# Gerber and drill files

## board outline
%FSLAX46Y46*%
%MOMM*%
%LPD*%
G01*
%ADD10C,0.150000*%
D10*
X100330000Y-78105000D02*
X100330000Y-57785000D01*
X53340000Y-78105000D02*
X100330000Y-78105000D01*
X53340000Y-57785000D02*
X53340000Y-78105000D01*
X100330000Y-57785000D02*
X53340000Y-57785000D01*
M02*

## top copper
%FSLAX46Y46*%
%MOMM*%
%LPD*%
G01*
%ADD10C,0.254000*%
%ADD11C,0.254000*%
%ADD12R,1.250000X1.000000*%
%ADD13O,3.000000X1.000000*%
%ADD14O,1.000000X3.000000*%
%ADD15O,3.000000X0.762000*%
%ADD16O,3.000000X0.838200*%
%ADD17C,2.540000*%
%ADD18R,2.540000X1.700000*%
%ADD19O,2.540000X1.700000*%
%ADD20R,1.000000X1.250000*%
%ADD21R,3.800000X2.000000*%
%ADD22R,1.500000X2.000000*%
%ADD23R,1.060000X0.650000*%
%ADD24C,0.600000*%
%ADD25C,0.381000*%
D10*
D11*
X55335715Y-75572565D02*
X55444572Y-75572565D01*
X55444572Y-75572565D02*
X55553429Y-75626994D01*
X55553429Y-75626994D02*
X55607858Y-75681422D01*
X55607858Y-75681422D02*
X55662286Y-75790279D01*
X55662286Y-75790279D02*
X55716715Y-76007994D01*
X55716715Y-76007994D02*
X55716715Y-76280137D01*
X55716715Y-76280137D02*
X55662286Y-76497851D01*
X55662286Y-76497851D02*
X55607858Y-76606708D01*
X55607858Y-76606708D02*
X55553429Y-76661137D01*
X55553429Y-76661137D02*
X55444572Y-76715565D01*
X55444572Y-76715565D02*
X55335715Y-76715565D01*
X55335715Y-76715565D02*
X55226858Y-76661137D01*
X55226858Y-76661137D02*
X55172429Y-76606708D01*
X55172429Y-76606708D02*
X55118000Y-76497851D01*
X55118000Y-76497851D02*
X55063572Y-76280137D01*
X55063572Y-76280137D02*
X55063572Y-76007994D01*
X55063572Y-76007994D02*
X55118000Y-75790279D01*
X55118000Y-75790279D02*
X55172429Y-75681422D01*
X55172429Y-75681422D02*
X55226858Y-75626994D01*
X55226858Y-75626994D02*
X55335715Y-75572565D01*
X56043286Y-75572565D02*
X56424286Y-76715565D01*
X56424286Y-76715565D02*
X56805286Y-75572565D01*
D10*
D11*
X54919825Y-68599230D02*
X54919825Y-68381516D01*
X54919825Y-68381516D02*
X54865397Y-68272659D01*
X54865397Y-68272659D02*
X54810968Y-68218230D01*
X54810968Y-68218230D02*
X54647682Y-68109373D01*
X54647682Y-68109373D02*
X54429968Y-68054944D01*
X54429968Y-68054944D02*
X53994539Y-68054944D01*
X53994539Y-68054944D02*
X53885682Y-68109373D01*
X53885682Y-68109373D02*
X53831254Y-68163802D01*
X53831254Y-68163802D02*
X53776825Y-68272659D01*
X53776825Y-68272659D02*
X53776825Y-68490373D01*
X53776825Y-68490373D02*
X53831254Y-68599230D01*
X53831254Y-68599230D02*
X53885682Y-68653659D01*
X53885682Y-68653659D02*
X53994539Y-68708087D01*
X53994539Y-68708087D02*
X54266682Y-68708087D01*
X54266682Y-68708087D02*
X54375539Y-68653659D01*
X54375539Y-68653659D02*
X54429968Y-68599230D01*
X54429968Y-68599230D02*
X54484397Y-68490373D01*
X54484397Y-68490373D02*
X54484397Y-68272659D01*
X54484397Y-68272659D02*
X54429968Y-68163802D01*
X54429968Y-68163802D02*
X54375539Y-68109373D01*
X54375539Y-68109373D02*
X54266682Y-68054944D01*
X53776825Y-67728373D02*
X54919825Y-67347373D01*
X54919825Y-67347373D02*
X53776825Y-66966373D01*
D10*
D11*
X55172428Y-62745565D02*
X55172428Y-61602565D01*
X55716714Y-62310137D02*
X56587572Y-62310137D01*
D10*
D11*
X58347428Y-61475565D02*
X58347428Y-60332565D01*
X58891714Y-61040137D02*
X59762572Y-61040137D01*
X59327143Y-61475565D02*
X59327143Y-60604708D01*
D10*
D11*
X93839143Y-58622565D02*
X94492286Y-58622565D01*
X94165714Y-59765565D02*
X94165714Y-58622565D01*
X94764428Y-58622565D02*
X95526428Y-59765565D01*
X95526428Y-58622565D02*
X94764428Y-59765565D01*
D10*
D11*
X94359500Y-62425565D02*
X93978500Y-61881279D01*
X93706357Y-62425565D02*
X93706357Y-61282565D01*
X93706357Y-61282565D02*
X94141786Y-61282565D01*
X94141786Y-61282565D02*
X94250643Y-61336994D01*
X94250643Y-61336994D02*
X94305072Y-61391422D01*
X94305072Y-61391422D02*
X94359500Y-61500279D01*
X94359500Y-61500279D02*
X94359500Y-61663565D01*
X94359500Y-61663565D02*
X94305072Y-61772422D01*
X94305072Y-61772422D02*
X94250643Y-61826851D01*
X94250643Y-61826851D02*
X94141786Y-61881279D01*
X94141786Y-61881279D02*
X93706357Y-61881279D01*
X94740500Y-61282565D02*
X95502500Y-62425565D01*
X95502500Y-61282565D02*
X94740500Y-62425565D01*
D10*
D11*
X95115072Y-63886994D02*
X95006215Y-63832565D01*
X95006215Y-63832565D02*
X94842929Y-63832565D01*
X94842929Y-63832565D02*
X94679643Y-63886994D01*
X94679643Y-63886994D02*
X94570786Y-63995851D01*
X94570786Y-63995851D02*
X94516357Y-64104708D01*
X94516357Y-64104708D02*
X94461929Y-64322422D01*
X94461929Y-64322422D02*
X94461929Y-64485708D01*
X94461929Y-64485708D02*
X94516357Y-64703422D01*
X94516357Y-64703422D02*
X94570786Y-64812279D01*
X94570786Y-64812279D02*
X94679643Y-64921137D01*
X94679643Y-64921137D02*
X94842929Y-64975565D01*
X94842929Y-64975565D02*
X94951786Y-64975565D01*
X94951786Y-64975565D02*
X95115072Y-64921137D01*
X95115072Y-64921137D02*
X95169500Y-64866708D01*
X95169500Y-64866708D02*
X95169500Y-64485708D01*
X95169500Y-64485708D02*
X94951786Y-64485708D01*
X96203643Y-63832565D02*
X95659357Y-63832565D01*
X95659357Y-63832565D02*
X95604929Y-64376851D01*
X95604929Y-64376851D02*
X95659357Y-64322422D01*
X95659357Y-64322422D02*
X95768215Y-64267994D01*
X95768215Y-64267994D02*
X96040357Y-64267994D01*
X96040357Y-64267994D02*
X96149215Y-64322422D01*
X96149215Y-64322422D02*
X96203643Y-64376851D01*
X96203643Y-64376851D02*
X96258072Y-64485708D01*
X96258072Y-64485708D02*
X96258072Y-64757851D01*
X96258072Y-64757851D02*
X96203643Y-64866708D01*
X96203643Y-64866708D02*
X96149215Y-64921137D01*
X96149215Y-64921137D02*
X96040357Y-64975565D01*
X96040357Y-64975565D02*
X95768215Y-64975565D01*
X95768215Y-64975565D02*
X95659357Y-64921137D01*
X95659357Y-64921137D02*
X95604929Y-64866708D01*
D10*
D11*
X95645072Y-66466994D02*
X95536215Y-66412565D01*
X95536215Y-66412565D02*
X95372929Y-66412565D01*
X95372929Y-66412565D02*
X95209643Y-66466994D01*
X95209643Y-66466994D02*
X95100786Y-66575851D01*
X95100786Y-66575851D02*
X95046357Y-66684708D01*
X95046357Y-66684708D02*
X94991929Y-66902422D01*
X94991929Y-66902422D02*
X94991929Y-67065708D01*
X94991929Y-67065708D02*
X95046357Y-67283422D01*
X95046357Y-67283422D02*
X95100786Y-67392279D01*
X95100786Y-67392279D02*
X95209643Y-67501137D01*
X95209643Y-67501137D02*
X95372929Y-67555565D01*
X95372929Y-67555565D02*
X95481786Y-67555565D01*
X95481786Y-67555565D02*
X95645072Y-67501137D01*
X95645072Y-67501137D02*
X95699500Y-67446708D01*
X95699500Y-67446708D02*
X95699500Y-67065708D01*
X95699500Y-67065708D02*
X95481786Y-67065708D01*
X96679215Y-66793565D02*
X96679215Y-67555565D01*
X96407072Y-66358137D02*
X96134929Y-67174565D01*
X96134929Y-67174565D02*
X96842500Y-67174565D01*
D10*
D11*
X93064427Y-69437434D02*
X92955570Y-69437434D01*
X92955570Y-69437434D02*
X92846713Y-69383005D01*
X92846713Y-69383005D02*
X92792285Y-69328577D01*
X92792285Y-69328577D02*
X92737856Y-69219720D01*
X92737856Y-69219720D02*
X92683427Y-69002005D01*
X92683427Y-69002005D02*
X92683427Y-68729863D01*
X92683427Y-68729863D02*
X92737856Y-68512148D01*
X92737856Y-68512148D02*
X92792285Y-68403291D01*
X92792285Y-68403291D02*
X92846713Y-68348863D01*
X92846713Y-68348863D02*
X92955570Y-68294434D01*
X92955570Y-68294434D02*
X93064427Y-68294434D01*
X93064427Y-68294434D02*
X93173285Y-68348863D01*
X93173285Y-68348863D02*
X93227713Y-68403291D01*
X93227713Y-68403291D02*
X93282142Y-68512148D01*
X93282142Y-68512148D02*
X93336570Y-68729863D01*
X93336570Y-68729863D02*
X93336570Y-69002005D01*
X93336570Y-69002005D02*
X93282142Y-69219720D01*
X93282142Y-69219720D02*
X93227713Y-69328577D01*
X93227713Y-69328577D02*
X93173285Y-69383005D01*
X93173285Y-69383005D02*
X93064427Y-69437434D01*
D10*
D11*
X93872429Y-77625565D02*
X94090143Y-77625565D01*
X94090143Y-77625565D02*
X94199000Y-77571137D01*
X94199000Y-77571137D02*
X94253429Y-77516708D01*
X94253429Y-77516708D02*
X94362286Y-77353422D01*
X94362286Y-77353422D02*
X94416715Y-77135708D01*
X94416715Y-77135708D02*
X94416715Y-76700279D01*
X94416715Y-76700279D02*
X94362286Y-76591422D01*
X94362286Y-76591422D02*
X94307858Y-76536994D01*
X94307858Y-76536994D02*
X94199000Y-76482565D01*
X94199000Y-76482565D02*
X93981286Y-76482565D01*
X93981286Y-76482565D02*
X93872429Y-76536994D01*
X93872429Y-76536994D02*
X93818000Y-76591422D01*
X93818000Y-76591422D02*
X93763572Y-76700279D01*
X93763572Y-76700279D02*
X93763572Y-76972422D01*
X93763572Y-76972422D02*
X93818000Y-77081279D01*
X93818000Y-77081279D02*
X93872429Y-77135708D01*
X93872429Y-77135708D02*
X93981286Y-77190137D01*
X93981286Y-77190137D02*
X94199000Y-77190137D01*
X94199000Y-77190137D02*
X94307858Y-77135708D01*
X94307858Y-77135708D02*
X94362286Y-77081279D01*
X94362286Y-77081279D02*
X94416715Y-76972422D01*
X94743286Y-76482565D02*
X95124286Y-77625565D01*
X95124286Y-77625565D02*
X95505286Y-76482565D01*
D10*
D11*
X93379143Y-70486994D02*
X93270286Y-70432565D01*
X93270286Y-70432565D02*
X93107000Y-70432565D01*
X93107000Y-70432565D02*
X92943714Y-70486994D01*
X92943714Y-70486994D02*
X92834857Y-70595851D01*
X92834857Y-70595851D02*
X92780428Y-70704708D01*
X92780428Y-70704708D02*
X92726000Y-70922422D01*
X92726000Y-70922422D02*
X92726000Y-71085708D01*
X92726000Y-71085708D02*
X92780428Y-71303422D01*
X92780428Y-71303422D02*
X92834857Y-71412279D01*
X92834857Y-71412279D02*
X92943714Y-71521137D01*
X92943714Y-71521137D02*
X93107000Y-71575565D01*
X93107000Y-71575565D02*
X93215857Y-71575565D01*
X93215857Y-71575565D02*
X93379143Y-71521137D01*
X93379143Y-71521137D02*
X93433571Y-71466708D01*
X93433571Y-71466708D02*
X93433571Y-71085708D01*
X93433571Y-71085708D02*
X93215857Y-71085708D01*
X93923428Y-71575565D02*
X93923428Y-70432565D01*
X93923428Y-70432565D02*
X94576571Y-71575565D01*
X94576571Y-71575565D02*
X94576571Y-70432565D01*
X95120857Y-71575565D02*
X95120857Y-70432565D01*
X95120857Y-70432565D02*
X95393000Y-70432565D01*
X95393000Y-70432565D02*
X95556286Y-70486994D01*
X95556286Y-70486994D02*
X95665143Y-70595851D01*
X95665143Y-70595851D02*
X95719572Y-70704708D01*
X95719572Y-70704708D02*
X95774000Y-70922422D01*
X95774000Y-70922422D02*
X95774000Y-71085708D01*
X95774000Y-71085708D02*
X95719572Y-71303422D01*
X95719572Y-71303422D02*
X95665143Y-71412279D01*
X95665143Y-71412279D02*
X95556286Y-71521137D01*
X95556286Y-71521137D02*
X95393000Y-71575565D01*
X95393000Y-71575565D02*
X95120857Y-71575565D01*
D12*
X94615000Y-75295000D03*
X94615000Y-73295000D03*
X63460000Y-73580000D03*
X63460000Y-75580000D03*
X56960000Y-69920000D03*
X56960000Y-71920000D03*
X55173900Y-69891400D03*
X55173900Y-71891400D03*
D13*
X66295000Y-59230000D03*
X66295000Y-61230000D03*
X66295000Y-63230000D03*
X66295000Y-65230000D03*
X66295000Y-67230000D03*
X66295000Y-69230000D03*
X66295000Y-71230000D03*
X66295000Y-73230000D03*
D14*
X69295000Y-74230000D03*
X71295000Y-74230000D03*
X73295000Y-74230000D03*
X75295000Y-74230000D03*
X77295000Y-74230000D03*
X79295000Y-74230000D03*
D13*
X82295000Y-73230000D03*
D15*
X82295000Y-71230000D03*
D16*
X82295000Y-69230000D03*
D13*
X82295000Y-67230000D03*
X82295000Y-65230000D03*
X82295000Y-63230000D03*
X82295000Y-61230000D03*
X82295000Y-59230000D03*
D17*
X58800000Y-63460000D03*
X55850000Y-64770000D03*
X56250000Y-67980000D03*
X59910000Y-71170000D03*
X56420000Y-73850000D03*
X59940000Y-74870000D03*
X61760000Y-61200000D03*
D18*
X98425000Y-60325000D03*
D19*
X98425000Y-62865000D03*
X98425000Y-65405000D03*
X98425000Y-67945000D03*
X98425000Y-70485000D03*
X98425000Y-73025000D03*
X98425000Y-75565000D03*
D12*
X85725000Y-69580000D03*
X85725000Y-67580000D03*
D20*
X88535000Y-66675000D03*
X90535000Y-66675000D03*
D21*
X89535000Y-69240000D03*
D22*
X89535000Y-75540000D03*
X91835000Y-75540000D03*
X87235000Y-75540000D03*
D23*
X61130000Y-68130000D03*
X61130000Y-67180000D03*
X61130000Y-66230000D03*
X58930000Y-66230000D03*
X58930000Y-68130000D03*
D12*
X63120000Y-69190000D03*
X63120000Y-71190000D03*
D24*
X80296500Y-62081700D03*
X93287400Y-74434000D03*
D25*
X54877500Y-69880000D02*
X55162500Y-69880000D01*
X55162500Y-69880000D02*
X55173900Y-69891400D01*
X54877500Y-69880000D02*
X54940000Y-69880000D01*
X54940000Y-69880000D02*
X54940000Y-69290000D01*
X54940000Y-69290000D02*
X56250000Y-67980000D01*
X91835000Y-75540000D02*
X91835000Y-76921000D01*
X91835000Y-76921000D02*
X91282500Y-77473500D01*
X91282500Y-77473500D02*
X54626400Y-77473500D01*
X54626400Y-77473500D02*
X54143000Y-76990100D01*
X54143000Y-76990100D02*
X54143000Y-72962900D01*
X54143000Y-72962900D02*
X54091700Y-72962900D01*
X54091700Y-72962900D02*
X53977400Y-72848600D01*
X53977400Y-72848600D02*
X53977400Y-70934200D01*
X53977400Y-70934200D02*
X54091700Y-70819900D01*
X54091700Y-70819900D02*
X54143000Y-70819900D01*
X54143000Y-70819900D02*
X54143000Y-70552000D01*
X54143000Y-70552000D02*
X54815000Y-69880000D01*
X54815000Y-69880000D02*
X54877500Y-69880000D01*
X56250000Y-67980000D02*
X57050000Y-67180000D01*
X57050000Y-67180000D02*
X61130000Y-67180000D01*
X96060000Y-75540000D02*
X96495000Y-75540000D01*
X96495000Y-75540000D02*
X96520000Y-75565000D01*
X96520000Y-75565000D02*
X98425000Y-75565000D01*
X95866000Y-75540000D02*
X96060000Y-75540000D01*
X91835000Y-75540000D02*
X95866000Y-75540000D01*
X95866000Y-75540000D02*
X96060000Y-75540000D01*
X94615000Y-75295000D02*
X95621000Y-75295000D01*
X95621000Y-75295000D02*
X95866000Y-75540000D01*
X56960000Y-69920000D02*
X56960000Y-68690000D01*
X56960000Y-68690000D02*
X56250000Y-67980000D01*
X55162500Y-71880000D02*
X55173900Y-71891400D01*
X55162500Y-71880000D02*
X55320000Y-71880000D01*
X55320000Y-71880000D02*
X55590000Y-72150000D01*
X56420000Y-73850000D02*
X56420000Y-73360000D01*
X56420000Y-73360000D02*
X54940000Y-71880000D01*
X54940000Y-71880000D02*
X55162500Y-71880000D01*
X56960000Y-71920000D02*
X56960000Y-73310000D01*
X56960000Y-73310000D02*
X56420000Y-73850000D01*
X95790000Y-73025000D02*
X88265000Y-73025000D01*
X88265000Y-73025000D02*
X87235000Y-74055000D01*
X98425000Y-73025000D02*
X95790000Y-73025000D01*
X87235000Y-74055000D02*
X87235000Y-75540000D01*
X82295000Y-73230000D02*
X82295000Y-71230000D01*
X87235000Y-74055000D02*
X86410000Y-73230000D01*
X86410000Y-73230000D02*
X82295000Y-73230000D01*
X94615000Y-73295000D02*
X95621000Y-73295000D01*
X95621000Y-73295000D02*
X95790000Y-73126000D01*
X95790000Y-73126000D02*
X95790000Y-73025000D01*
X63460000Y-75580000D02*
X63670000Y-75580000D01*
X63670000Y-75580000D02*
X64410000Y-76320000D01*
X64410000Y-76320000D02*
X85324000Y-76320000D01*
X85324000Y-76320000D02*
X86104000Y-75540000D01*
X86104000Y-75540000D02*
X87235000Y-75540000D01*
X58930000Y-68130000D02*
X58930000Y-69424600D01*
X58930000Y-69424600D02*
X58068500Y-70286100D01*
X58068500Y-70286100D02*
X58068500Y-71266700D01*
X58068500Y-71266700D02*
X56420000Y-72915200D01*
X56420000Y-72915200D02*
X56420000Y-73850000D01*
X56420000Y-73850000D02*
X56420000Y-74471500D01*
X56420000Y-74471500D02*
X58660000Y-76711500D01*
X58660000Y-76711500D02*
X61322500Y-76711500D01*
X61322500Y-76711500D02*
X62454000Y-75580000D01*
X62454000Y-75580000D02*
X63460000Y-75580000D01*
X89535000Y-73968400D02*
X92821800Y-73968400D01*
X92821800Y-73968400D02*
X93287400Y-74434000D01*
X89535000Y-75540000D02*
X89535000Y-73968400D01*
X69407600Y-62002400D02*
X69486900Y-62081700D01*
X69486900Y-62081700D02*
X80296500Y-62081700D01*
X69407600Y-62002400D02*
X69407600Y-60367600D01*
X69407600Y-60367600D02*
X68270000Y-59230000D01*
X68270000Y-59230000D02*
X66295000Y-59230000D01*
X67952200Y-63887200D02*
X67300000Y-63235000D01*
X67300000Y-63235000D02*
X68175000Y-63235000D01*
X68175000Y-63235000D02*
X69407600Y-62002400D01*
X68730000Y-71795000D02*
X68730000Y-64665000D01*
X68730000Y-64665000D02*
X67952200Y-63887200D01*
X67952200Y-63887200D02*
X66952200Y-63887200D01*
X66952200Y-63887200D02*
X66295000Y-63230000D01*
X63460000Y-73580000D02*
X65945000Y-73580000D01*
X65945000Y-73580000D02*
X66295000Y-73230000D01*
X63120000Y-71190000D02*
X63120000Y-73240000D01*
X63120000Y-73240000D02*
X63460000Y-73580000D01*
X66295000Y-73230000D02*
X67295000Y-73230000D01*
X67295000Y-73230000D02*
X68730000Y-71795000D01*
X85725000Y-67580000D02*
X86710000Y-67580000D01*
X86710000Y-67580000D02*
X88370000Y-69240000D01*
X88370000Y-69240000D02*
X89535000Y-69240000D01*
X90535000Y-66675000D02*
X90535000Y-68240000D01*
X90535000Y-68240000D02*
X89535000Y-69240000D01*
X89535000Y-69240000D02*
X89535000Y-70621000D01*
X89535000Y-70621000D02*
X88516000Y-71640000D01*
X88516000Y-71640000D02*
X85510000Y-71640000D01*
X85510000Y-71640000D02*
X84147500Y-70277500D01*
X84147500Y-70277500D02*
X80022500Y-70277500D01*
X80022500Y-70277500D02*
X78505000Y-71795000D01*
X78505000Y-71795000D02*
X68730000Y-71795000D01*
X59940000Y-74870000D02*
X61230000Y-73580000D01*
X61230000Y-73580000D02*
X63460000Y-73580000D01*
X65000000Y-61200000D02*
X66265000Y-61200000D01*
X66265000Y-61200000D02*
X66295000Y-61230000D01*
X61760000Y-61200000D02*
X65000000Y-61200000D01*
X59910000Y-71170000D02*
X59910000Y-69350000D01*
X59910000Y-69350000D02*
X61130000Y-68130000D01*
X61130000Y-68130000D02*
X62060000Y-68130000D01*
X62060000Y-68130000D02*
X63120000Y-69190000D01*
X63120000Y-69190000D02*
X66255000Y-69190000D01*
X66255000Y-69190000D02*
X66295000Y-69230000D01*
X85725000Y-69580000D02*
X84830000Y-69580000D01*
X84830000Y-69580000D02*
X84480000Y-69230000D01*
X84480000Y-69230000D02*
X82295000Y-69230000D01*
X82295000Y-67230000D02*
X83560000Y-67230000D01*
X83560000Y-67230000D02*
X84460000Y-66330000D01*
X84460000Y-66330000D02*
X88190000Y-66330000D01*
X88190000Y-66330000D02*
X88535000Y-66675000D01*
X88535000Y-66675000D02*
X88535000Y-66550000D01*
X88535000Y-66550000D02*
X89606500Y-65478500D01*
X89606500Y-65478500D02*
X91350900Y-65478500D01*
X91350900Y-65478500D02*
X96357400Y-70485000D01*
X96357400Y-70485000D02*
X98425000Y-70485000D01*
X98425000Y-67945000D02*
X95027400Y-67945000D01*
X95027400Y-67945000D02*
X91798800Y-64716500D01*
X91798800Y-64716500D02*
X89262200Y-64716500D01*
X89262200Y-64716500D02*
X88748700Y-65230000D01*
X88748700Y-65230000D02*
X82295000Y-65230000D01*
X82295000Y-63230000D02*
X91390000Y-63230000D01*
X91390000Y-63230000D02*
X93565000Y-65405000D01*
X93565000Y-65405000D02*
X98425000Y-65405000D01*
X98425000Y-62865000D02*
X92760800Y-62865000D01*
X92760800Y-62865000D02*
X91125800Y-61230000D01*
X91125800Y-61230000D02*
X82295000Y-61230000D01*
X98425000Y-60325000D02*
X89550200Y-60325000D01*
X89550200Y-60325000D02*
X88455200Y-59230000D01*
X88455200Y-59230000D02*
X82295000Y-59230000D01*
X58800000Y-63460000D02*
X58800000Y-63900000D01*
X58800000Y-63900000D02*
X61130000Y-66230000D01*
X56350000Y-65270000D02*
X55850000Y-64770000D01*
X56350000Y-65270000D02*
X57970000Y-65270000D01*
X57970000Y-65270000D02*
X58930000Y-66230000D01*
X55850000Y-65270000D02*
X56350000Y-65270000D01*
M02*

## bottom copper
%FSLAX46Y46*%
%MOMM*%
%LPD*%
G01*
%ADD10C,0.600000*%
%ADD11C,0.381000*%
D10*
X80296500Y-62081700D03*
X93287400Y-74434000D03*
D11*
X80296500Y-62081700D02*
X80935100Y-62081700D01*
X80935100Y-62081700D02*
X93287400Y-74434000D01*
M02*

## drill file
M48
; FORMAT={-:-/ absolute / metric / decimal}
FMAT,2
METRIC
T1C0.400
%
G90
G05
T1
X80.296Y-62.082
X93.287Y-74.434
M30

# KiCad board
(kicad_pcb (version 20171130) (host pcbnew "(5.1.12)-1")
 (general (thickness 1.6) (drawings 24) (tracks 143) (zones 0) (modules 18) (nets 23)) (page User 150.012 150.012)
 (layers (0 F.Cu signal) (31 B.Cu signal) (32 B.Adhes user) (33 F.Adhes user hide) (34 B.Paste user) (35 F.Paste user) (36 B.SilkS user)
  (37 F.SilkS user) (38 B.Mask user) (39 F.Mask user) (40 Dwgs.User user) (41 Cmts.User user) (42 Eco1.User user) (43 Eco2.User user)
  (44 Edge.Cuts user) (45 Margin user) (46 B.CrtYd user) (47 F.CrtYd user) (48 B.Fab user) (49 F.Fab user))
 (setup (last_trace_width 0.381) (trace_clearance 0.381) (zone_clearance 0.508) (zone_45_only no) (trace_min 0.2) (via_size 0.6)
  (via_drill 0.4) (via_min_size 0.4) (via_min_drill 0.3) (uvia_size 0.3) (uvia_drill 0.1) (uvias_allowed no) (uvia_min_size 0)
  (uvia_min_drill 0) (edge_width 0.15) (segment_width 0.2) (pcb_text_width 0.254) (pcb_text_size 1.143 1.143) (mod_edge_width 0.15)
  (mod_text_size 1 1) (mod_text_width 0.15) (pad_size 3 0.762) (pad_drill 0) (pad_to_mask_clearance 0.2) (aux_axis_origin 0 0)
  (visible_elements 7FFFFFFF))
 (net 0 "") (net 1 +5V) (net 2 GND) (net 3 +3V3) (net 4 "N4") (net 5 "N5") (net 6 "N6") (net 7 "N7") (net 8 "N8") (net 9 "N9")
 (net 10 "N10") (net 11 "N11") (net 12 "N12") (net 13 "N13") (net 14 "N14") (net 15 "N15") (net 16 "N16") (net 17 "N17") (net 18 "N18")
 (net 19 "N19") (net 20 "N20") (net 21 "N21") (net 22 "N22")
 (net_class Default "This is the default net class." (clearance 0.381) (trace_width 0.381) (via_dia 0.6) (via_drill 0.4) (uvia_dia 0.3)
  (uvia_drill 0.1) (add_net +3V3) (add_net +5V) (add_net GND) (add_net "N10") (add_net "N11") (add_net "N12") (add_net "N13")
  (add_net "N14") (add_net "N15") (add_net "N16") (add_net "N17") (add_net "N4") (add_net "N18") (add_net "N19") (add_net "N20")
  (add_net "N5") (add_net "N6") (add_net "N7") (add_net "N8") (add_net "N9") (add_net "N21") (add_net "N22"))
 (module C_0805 (layer F.Cu) (at 94.615 74.295 90)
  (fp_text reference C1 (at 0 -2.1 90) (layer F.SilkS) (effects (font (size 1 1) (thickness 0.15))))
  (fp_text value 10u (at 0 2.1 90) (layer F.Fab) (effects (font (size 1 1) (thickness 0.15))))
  (pad 1 smd rect (at -1 0 90) (size 1 1.25) (layers F.Cu F.Paste F.Mask) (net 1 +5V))
  (pad 2 smd rect (at 1 0 90) (size 1 1.25) (layers F.Cu F.Paste F.Mask) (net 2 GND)))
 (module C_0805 (layer F.Cu) (at 63.46 74.58 270)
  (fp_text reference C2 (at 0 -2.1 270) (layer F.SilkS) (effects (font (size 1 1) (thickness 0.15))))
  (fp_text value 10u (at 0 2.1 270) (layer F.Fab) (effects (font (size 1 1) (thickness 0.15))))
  (pad 1 smd rect (at -1 0 270) (size 1 1.25) (layers F.Cu F.Paste F.Mask) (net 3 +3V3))
  (pad 2 smd rect (at 1 0 270) (size 1 1.25) (layers F.Cu F.Paste F.Mask) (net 2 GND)))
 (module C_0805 (layer F.Cu) (at 56.96 70.92 270)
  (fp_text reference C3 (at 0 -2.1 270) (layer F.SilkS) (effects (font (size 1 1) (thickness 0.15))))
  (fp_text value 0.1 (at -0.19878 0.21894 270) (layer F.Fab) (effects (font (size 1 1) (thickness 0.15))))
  (pad 1 smd rect (at -1 0 270) (size 1 1.25) (layers F.Cu F.Paste F.Mask) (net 1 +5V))
  (pad 2 smd rect (at 1 0 270) (size 1 1.25) (layers F.Cu F.Paste F.Mask) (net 2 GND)))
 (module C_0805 (layer F.Cu) (at 55.1739 70.8914 270)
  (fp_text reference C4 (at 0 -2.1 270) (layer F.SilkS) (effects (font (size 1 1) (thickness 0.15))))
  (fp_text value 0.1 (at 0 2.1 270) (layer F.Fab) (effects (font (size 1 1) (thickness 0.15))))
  (pad 1 smd rect (at -1 0 270) (size 1 1.25) (layers F.Cu F.Paste F.Mask) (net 1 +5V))
  (pad 2 smd rect (at 1 0 270) (size 1 1.25) (layers F.Cu F.Paste F.Mask) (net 2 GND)))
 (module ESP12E (layer F.Cu) (at 74.295 62.23)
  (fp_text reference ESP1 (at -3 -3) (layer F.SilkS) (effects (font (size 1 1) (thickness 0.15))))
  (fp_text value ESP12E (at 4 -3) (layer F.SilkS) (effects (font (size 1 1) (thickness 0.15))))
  (pad 1 smd oval (at -8 -3) (size 3 1) (layers F.Cu F.Paste F.Mask) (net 3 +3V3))
  (pad 2 smd oval (at -8 -1) (size 3 1) (layers F.Cu F.Paste F.Mask) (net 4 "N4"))
  (pad 3 smd oval (at -8 1) (size 3 1) (layers F.Cu F.Paste F.Mask) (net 3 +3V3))
  (pad 4 smd oval (at -8 3) (size 3 1) (layers F.Cu F.Paste F.Mask) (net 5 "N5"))
  (pad 5 smd oval (at -8 5) (size 3 1) (layers F.Cu F.Paste F.Mask) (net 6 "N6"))
  (pad 6 smd oval (at -8 7) (size 3 1) (layers F.Cu F.Paste F.Mask) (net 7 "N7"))
  (pad 7 smd oval (at -8 9) (size 3 1) (layers F.Cu F.Paste F.Mask) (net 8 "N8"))
  (pad 8 smd oval (at -8 11) (size 3 1) (layers F.Cu F.Paste F.Mask) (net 3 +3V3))
  (pad 9 smd oval (at -5 12 90) (size 3 1) (layers F.Cu F.Paste F.Mask) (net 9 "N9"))
  (pad 10 smd oval (at -3 12 90) (size 3 1) (layers F.Cu F.Paste F.Mask) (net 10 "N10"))
  (pad 11 smd oval (at -1 12 90) (size 3 1) (layers F.Cu F.Paste F.Mask) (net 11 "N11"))
  (pad 12 smd oval (at 1 12 90) (size 3 1) (layers F.Cu F.Paste F.Mask) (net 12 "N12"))
  (pad 13 smd oval (at 3 12 90) (size 3 1) (layers F.Cu F.Paste F.Mask) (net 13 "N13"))
  (pad 14 smd oval (at 5 12 90) (size 3 1) (layers F.Cu F.Paste F.Mask) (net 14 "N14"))
  (pad 15 smd oval (at 8 11 180) (size 3 1) (layers F.Cu F.Paste F.Mask) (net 2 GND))
  (pad 16 smd oval (at 8 9 180) (size 3 0.762) (layers F.Cu F.Paste F.Mask) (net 2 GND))
  (pad 17 smd oval (at 8 7 180) (size 3 0.8382) (layers F.Cu F.Paste F.Mask) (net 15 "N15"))
  (pad 18 smd oval (at 8 5 180) (size 3 1) (layers F.Cu F.Paste F.Mask) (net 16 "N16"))
  (pad 19 smd oval (at 8 3 180) (size 3 1) (layers F.Cu F.Paste F.Mask) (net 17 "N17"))
  (pad 20 smd oval (at 8 1 180) (size 3 1) (layers F.Cu F.Paste F.Mask) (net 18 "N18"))
  (pad 21 smd oval (at 8 -1 180) (size 3 1) (layers F.Cu F.Paste F.Mask) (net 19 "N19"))
  (pad 22 smd oval (at 8 -3 180) (size 3 1) (layers F.Cu F.Paste F.Mask) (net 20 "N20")))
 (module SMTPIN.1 (layer F.Cu) (at 58.8 63.46)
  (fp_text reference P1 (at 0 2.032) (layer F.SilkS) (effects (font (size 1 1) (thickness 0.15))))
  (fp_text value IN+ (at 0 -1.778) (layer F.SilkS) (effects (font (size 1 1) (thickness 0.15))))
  (pad 1 smd circle (at 0 0) (size 2.54 2.54) (layers F.Cu F.Paste F.Mask) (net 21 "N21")))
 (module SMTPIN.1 (layer F.Cu) (at 55.85 64.77)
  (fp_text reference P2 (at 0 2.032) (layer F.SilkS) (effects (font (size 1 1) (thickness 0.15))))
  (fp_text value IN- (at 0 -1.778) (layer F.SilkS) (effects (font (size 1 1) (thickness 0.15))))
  (pad 1 smd circle (at 0 0) (size 2.54 2.54) (layers F.Cu F.Paste F.Mask) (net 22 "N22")))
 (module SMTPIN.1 (layer F.Cu) (at 56.25 67.98)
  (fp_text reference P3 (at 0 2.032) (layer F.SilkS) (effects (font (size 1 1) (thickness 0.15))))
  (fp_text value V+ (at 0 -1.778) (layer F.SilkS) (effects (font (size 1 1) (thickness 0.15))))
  (pad 1 smd circle (at 0 0) (size 2.54 2.54) (layers F.Cu F.Paste F.Mask) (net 1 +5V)))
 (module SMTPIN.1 (layer F.Cu) (at 59.91 71.17)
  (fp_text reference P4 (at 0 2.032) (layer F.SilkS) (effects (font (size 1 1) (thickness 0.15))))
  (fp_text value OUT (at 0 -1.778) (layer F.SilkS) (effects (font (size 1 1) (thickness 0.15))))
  (pad 1 smd circle (at 0 0) (size 2.54 2.54) (layers F.Cu F.Paste F.Mask) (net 7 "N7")))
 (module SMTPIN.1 (layer F.Cu) (at 56.42 73.85)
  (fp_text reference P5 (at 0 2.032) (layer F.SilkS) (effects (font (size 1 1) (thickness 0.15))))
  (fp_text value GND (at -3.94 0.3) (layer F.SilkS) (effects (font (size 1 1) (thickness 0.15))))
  (pad 1 smd circle (at 0 0) (size 2.54 2.54) (layers F.Cu F.Paste F.Mask) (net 2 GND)))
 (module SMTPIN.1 (layer F.Cu) (at 59.94 74.87)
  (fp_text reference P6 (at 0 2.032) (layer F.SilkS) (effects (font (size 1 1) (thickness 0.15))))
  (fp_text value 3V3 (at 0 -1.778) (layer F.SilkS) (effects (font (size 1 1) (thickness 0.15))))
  (pad 1 smd circle (at 0 0) (size 2.54 2.54) (layers F.Cu F.Paste F.Mask) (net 3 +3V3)))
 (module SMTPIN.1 (layer F.Cu) (at 61.76 61.2)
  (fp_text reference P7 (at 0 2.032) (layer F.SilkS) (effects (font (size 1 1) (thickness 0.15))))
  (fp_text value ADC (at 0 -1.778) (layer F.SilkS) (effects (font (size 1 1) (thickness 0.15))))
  (pad 1 smd circle (at 0 0) (size 2.54 2.54) (layers F.Cu F.Paste F.Mask) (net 4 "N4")))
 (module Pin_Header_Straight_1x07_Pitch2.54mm (layer F.Cu) (at 98.425 60.325)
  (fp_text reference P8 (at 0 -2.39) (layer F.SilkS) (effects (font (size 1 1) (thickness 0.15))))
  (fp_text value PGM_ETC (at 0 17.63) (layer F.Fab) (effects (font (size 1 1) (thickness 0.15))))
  (pad 1 smd rect (at 0 0) (size 2.54 1.7) (layers F.Cu F.Paste F.Mask) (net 20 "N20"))
  (pad 2 smd oval (at 0 2.54) (size 2.54 1.7) (layers F.Cu F.Paste F.Mask) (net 19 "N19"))
  (pad 3 smd oval (at 0 5.08) (size 2.54 1.7) (layers F.Cu F.Paste F.Mask) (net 18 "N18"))
  (pad 4 smd oval (at 0 7.62) (size 2.54 1.7) (layers F.Cu F.Paste F.Mask) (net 17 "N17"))
  (pad 5 smd oval (at 0 10.16) (size 2.54 1.7) (layers F.Cu F.Paste F.Mask) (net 16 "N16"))
  (pad 6 smd oval (at 0 12.7) (size 2.54 1.7) (layers F.Cu F.Paste F.Mask) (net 2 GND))
  (pad 7 smd oval (at 0 15.24) (size 2.54 1.7) (layers F.Cu F.Paste F.Mask) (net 1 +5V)))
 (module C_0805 (layer F.Cu) (at 85.725 68.58 90)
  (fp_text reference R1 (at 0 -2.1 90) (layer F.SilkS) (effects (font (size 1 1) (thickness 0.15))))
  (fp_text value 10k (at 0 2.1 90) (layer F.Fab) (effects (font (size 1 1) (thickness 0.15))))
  (pad 1 smd rect (at -1 0 90) (size 1 1.25) (layers F.Cu F.Paste F.Mask) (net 15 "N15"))
  (pad 2 smd rect (at 1 0 90) (size 1 1.25) (layers F.Cu F.Paste F.Mask) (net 3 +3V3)))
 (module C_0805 (layer F.Cu) (at 89.535 66.675)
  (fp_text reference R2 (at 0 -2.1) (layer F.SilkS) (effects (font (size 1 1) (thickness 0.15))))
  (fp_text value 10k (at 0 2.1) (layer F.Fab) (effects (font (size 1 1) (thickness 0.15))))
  (pad 1 smd rect (at -1 0) (size 1 1.25) (layers F.Cu F.Paste F.Mask) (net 16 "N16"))
  (pad 2 smd rect (at 1 0) (size 1 1.25) (layers F.Cu F.Paste F.Mask) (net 3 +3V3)))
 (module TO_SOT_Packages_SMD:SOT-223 (layer F.Cu) (at 89.535 72.39 90)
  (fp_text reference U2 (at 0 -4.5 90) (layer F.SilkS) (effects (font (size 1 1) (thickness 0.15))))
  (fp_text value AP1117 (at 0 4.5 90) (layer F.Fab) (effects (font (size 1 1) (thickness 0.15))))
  (pad 4 smd rect (at 3.15 0 90) (size 2 3.8) (layers F.Cu F.Paste F.Mask) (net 3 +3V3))
  (pad 2 smd rect (at -3.15 0 90) (size 2 1.5) (layers F.Cu F.Paste F.Mask) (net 3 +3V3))
  (pad 3 smd rect (at -3.15 2.3 90) (size 2 1.5) (layers F.Cu F.Paste F.Mask) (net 1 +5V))
  (pad 1 smd rect (at -3.15 -2.3 90) (size 2 1.5) (layers F.Cu F.Paste F.Mask) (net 2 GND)))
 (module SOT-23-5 (layer F.Cu) (at 60.03 67.18 180)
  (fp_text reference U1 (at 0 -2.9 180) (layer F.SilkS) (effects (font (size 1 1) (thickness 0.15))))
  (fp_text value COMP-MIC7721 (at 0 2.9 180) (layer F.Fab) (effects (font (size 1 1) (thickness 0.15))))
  (pad 1 smd rect (at -1.1 -0.95 180) (size 1.06 0.65) (layers F.Cu F.Paste F.Mask) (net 7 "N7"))
  (pad 2 smd rect (at -1.1 0 180) (size 1.06 0.65) (layers F.Cu F.Paste F.Mask) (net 1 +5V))
  (pad 3 smd rect (at -1.1 0.95 180) (size 1.06 0.65) (layers F.Cu F.Paste F.Mask) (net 21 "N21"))
  (pad 4 smd rect (at 1.1 0.95 180) (size 1.06 0.65) (layers F.Cu F.Paste F.Mask) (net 22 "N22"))
  (pad 5 smd rect (at 1.1 -0.95 180) (size 1.06 0.65) (layers F.Cu F.Paste F.Mask) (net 2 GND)))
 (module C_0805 (layer F.Cu) (at 63.12 70.19 270)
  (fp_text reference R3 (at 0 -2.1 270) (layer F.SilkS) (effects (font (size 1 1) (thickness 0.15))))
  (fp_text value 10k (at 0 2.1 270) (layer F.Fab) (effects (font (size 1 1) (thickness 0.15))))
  (pad 1 smd rect (at -1 0 270) (size 1 1.25) (layers F.Cu F.Paste F.Mask) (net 7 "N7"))
  (pad 2 smd rect (at 1 0 270) (size 1 1.25) (layers F.Cu F.Paste F.Mask) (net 3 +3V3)))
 (gr_line (start 100.33 78.105) (end 100.33 57.785) (layer Edge.Cuts) (width 0.15))
 (gr_line (start 53.34 78.105) (end 100.33 78.105) (layer Edge.Cuts) (width 0.15))
 (gr_line (start 53.34 57.785) (end 53.34 78.105) (layer Edge.Cuts) (width 0.15))
 (gr_line (start 100.33 57.785) (end 53.34 57.785) (layer Edge.Cuts) (width 0.15))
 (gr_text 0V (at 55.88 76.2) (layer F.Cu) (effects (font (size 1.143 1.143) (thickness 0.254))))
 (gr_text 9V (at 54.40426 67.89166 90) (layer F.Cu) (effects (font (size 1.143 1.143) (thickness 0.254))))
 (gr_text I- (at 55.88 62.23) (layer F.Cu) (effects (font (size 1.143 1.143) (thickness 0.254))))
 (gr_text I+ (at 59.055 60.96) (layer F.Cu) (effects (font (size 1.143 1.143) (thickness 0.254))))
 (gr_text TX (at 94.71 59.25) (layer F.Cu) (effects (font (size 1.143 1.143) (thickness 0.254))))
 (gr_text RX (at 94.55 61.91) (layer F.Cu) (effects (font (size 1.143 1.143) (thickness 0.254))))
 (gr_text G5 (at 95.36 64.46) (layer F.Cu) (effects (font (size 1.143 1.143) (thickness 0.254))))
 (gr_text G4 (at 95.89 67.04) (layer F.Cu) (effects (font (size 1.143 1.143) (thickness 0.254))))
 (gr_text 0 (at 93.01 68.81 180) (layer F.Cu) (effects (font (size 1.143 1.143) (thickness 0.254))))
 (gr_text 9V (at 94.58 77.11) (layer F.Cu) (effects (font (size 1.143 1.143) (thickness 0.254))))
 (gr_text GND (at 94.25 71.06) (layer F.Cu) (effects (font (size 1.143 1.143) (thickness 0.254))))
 (segment (start 54.8775 69.88) (end 55.1625 69.88) (width 0.381) (layer F.Cu) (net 1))
 (segment (start 55.1625 69.88) (end 55.1739 69.8914) (width 0.381) (layer F.Cu) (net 1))
 (segment (start 54.8775 69.88) (end 54.94 69.88) (width 0.381) (layer F.Cu) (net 1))
 (segment (start 54.94 69.88) (end 54.94 69.29) (width 0.381) (layer F.Cu) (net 1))
 (segment (start 54.94 69.29) (end 56.25 67.98) (width 0.381) (layer F.Cu) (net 1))
 (segment (start 91.835 75.54) (end 91.835 76.921) (width 0.381) (layer F.Cu) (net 1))
 (segment (start 91.835 76.921) (end 91.2825 77.4735) (width 0.381) (layer F.Cu) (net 1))
 (segment (start 91.2825 77.4735) (end 54.6264 77.4735) (width 0.381) (layer F.Cu) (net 1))
 (segment (start 54.6264 77.4735) (end 54.143 76.9901) (width 0.381) (layer F.Cu) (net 1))
 (segment (start 54.143 76.9901) (end 54.143 72.9629) (width 0.381) (layer F.Cu) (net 1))
 (segment (start 54.143 72.9629) (end 54.0917 72.9629) (width 0.381) (layer F.Cu) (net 1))
 (segment (start 54.0917 72.9629) (end 53.9774 72.8486) (width 0.381) (layer F.Cu) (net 1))
 (segment (start 53.9774 72.8486) (end 53.9774 70.9342) (width 0.381) (layer F.Cu) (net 1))
 (segment (start 53.9774 70.9342) (end 54.0917 70.8199) (width 0.381) (layer F.Cu) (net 1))
 (segment (start 54.0917 70.8199) (end 54.143 70.8199) (width 0.381) (layer F.Cu) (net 1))
 (segment (start 54.143 70.8199) (end 54.143 70.552) (width 0.381) (layer F.Cu) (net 1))
 (segment (start 54.143 70.552) (end 54.815 69.88) (width 0.381) (layer F.Cu) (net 1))
 (segment (start 54.815 69.88) (end 54.8775 69.88) (width 0.381) (layer F.Cu) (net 1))
 (segment (start 56.25 67.98) (end 57.05 67.18) (width 0.381) (layer F.Cu) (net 1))
 (segment (start 57.05 67.18) (end 61.13 67.18) (width 0.381) (layer F.Cu) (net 1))
 (segment (start 96.06 75.54) (end 96.495 75.54) (width 0.381) (layer F.Cu) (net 1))
 (segment (start 96.495 75.54) (end 96.52 75.565) (width 0.381) (layer F.Cu) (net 1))
 (segment (start 96.52 75.565) (end 98.425 75.565) (width 0.381) (layer F.Cu) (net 1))
 (segment (start 95.866 75.54) (end 96.06 75.54) (width 0.381) (layer F.Cu) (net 1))
 (segment (start 91.835 75.54) (end 95.866 75.54) (width 0.381) (layer F.Cu) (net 1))
 (segment (start 95.866 75.54) (end 96.06 75.54) (width 0.381) (layer F.Cu) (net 1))
 (segment (start 94.615 75.295) (end 95.621 75.295) (width 0.381) (layer F.Cu) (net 1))
 (segment (start 95.621 75.295) (end 95.866 75.54) (width 0.381) (layer F.Cu) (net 1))
 (segment (start 56.96 69.92) (end 56.96 68.69) (width 0.381) (layer F.Cu) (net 1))
 (segment (start 56.96 68.69) (end 56.25 67.98) (width 0.381) (layer F.Cu) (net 1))
 (segment (start 55.1625 71.88) (end 55.1739 71.8914) (width 0.381) (layer F.Cu) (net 2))
 (segment (start 55.1625 71.88) (end 55.32 71.88) (width 0.381) (layer F.Cu) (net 2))
 (segment (start 55.32 71.88) (end 55.59 72.15) (width 0.381) (layer F.Cu) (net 2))
 (segment (start 56.42 73.85) (end 56.42 73.36) (width 0.381) (layer F.Cu) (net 2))
 (segment (start 56.42 73.36) (end 54.94 71.88) (width 0.381) (layer F.Cu) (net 2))
 (segment (start 54.94 71.88) (end 55.1625 71.88) (width 0.381) (layer F.Cu) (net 2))
 (segment (start 56.96 71.92) (end 56.96 73.31) (width 0.381) (layer F.Cu) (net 2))
 (segment (start 56.96 73.31) (end 56.42 73.85) (width 0.381) (layer F.Cu) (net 2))
 (segment (start 95.79 73.025) (end 88.265 73.025) (width 0.381) (layer F.Cu) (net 2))
 (segment (start 88.265 73.025) (end 87.235 74.055) (width 0.381) (layer F.Cu) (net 2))
 (segment (start 98.425 73.025) (end 95.79 73.025) (width 0.381) (layer F.Cu) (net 2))
 (segment (start 87.235 74.055) (end 87.235 75.54) (width 0.381) (layer F.Cu) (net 2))
 (segment (start 82.295 73.23) (end 82.295 71.23) (width 0.381) (layer F.Cu) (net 2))
 (segment (start 87.235 74.055) (end 86.41 73.23) (width 0.381) (layer F.Cu) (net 2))
 (segment (start 86.41 73.23) (end 82.295 73.23) (width 0.381) (layer F.Cu) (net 2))
 (segment (start 94.615 73.295) (end 95.621 73.295) (width 0.381) (layer F.Cu) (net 2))
 (segment (start 95.621 73.295) (end 95.79 73.126) (width 0.381) (layer F.Cu) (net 2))
 (segment (start 95.79 73.126) (end 95.79 73.025) (width 0.381) (layer F.Cu) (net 2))
 (segment (start 63.46 75.58) (end 63.67 75.58) (width 0.381) (layer F.Cu) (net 2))
 (segment (start 63.67 75.58) (end 64.41 76.32) (width 0.381) (layer F.Cu) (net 2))
 (segment (start 64.41 76.32) (end 85.324 76.32) (width 0.381) (layer F.Cu) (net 2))
 (segment (start 85.324 76.32) (end 86.104 75.54) (width 0.381) (layer F.Cu) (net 2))
 (segment (start 86.104 75.54) (end 87.235 75.54) (width 0.381) (layer F.Cu) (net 2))
 (segment (start 58.93 68.13) (end 58.93 69.4246) (width 0.381) (layer F.Cu) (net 2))
 (segment (start 58.93 69.4246) (end 58.0685 70.2861) (width 0.381) (layer F.Cu) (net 2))
 (segment (start 58.0685 70.2861) (end 58.0685 71.2667) (width 0.381) (layer F.Cu) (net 2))
 (segment (start 58.0685 71.2667) (end 56.42 72.9152) (width 0.381) (layer F.Cu) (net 2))
 (segment (start 56.42 72.9152) (end 56.42 73.85) (width 0.381) (layer F.Cu) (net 2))
 (segment (start 56.42 73.85) (end 56.42 74.4715) (width 0.381) (layer F.Cu) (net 2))
 (segment (start 56.42 74.4715) (end 58.66 76.7115) (width 0.381) (layer F.Cu) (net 2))
 (segment (start 58.66 76.7115) (end 61.3225 76.7115) (width 0.381) (layer F.Cu) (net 2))
 (segment (start 61.3225 76.7115) (end 62.454 75.58) (width 0.381) (layer F.Cu) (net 2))
 (segment (start 62.454 75.58) (end 63.46 75.58) (width 0.381) (layer F.Cu) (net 2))
 (segment (start 89.535 73.9684) (end 92.8218 73.9684) (width 0.381) (layer F.Cu) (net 3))
 (segment (start 92.8218 73.9684) (end 93.2874 74.434) (width 0.381) (layer F.Cu) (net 3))
 (segment (start 80.2965 62.0817) (end 80.9351 62.0817) (width 0.381) (layer B.Cu) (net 3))
 (segment (start 80.9351 62.0817) (end 93.2874 74.434) (width 0.381) (layer B.Cu) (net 3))
 (segment (start 89.535 75.54) (end 89.535 73.9684) (width 0.381) (layer F.Cu) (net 3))
 (segment (start 69.4076 62.0024) (end 69.4869 62.0817) (width 0.381) (layer F.Cu) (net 3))
 (segment (start 69.4869 62.0817) (end 80.2965 62.0817) (width 0.381) (layer F.Cu) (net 3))
 (segment (start 69.4076 62.0024) (end 69.4076 60.3676) (width 0.381) (layer F.Cu) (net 3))
 (segment (start 69.4076 60.3676) (end 68.27 59.23) (width 0.381) (layer F.Cu) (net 3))
 (segment (start 68.27 59.23) (end 66.295 59.23) (width 0.381) (layer F.Cu) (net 3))
 (segment (start 67.9522 63.8872) (end 67.3 63.235) (width 0.381) (layer F.Cu) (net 3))
 (segment (start 67.3 63.235) (end 68.175 63.235) (width 0.381) (layer F.Cu) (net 3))
 (segment (start 68.175 63.235) (end 69.4076 62.0024) (width 0.381) (layer F.Cu) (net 3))
 (segment (start 68.73 71.795) (end 68.73 64.665) (width 0.381) (layer F.Cu) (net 3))
 (segment (start 68.73 64.665) (end 67.9522 63.8872) (width 0.381) (layer F.Cu) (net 3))
 (segment (start 67.9522 63.8872) (end 66.9522 63.8872) (width 0.381) (layer F.Cu) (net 3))
 (segment (start 66.9522 63.8872) (end 66.295 63.23) (width 0.381) (layer F.Cu) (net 3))
 (segment (start 63.46 73.58) (end 65.945 73.58) (width 0.381) (layer F.Cu) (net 3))
 (segment (start 65.945 73.58) (end 66.295 73.23) (width 0.381) (layer F.Cu) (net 3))
 (segment (start 63.12 71.19) (end 63.12 73.24) (width 0.381) (layer F.Cu) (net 3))
 (segment (start 63.12 73.24) (end 63.46 73.58) (width 0.381) (layer F.Cu) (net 3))
 (segment (start 66.295 73.23) (end 67.295 73.23) (width 0.381) (layer F.Cu) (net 3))
 (segment (start 67.295 73.23) (end 68.73 71.795) (width 0.381) (layer F.Cu) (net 3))
 (segment (start 85.725 67.58) (end 86.71 67.58) (width 0.381) (layer F.Cu) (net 3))
 (segment (start 86.71 67.58) (end 88.37 69.24) (width 0.381) (layer F.Cu) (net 3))
 (segment (start 88.37 69.24) (end 89.535 69.24) (width 0.381) (layer F.Cu) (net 3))
 (segment (start 90.535 66.675) (end 90.535 68.24) (width 0.381) (layer F.Cu) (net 3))
 (segment (start 90.535 68.24) (end 89.535 69.24) (width 0.381) (layer F.Cu) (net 3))
 (segment (start 89.535 69.24) (end 89.535 70.621) (width 0.381) (layer F.Cu) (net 3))
 (segment (start 89.535 70.621) (end 88.516 71.64) (width 0.381) (layer F.Cu) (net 3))
 (segment (start 88.516 71.64) (end 85.51 71.64) (width 0.381) (layer F.Cu) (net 3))
 (segment (start 85.51 71.64) (end 84.1475 70.2775) (width 0.381) (layer F.Cu) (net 3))
 (segment (start 84.1475 70.2775) (end 80.0225 70.2775) (width 0.381) (layer F.Cu) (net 3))
 (segment (start 80.0225 70.2775) (end 78.505 71.795) (width 0.381) (layer F.Cu) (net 3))
 (segment (start 78.505 71.795) (end 68.73 71.795) (width 0.381) (layer F.Cu) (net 3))
 (segment (start 59.94 74.87) (end 61.23 73.58) (width 0.381) (layer F.Cu) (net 3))
 (segment (start 61.23 73.58) (end 63.46 73.58) (width 0.381) (layer F.Cu) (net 3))
 (via (at 80.2965 62.0817) (size 0.6) (layers F.Cu B.Cu) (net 3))
 (via (at 93.2874 74.434) (size 0.6) (layers F.Cu B.Cu) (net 3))
 (segment (start 65 61.2) (end 66.265 61.2) (width 0.381) (layer F.Cu) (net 4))
 (segment (start 66.265 61.2) (end 66.295 61.23) (width 0.381) (layer F.Cu) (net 4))
 (segment (start 61.76 61.2) (end 65 61.2) (width 0.381) (layer F.Cu) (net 4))
 (segment (start 59.91 71.17) (end 59.91 69.35) (width 0.381) (layer F.Cu) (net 7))
 (segment (start 59.91 69.35) (end 61.13 68.13) (width 0.381) (layer F.Cu) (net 7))
 (segment (start 61.13 68.13) (end 62.06 68.13) (width 0.381) (layer F.Cu) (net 7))
 (segment (start 62.06 68.13) (end 63.12 69.19) (width 0.381) (layer F.Cu) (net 7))
 (segment (start 63.12 69.19) (end 66.255 69.19) (width 0.381) (layer F.Cu) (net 7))
 (segment (start 66.255 69.19) (end 66.295 69.23) (width 0.381) (layer F.Cu) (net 7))
 (segment (start 85.725 69.58) (end 84.83 69.58) (width 0.381) (layer F.Cu) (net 15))
 (segment (start 84.83 69.58) (end 84.48 69.23) (width 0.381) (layer F.Cu) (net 15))
 (segment (start 84.48 69.23) (end 82.295 69.23) (width 0.381) (layer F.Cu) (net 15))
 (segment (start 82.295 67.23) (end 83.56 67.23) (width 0.381) (layer F.Cu) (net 16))
 (segment (start 83.56 67.23) (end 84.46 66.33) (width 0.381) (layer F.Cu) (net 16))
 (segment (start 84.46 66.33) (end 88.19 66.33) (width 0.381) (layer F.Cu) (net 16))
 (segment (start 88.19 66.33) (end 88.535 66.675) (width 0.381) (layer F.Cu) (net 16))
 (segment (start 88.535 66.675) (end 88.535 66.55) (width 0.381) (layer F.Cu) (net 16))
 (segment (start 88.535 66.55) (end 89.6065 65.4785) (width 0.381) (layer F.Cu) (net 16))
 (segment (start 89.6065 65.4785) (end 91.3509 65.4785) (width 0.381) (layer F.Cu) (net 16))
 (segment (start 91.3509 65.4785) (end 96.3574 70.485) (width 0.381) (layer F.Cu) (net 16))
 (segment (start 96.3574 70.485) (end 98.425 70.485) (width 0.381) (layer F.Cu) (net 16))
 (segment (start 98.425 67.945) (end 95.0274 67.945) (width 0.381) (layer F.Cu) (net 17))
 (segment (start 95.0274 67.945) (end 91.7988 64.7165) (width 0.381) (layer F.Cu) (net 17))
 (segment (start 91.7988 64.7165) (end 89.2622 64.7165) (width 0.381) (layer F.Cu) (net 17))
 (segment (start 89.2622 64.7165) (end 88.7487 65.23) (width 0.381) (layer F.Cu) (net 17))
 (segment (start 88.7487 65.23) (end 82.295 65.23) (width 0.381) (layer F.Cu) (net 17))
 (segment (start 82.295 63.23) (end 91.39 63.23) (width 0.381) (layer F.Cu) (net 18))
 (segment (start 91.39 63.23) (end 93.565 65.405) (width 0.381) (layer F.Cu) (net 18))
 (segment (start 93.565 65.405) (end 98.425 65.405) (width 0.381) (layer F.Cu) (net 18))
 (segment (start 98.425 62.865) (end 92.7608 62.865) (width 0.381) (layer F.Cu) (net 19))
 (segment (start 92.7608 62.865) (end 91.1258 61.23) (width 0.381) (layer F.Cu) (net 19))
 (segment (start 91.1258 61.23) (end 82.295 61.23) (width 0.381) (layer F.Cu) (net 19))
 (segment (start 98.425 60.325) (end 89.5502 60.325) (width 0.381) (layer F.Cu) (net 20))
 (segment (start 89.5502 60.325) (end 88.4552 59.23) (width 0.381) (layer F.Cu) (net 20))
 (segment (start 88.4552 59.23) (end 82.295 59.23) (width 0.381) (layer F.Cu) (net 20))
 (segment (start 58.8 63.46) (end 58.8 63.9) (width 0.381) (layer F.Cu) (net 21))
 (segment (start 58.8 63.9) (end 61.13 66.23) (width 0.381) (layer F.Cu) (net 21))
 (segment (start 56.35 65.27) (end 55.85 64.77) (width 0.381) (layer F.Cu) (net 22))
 (segment (start 56.35 65.27) (end 57.97 65.27) (width 0.381) (layer F.Cu) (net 22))
 (segment (start 57.97 65.27) (end 58.93 66.23) (width 0.381) (layer F.Cu) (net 22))
 (segment (start 55.85 65.27) (end 56.35 65.27) (width 0.381) (layer F.Cu) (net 22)))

